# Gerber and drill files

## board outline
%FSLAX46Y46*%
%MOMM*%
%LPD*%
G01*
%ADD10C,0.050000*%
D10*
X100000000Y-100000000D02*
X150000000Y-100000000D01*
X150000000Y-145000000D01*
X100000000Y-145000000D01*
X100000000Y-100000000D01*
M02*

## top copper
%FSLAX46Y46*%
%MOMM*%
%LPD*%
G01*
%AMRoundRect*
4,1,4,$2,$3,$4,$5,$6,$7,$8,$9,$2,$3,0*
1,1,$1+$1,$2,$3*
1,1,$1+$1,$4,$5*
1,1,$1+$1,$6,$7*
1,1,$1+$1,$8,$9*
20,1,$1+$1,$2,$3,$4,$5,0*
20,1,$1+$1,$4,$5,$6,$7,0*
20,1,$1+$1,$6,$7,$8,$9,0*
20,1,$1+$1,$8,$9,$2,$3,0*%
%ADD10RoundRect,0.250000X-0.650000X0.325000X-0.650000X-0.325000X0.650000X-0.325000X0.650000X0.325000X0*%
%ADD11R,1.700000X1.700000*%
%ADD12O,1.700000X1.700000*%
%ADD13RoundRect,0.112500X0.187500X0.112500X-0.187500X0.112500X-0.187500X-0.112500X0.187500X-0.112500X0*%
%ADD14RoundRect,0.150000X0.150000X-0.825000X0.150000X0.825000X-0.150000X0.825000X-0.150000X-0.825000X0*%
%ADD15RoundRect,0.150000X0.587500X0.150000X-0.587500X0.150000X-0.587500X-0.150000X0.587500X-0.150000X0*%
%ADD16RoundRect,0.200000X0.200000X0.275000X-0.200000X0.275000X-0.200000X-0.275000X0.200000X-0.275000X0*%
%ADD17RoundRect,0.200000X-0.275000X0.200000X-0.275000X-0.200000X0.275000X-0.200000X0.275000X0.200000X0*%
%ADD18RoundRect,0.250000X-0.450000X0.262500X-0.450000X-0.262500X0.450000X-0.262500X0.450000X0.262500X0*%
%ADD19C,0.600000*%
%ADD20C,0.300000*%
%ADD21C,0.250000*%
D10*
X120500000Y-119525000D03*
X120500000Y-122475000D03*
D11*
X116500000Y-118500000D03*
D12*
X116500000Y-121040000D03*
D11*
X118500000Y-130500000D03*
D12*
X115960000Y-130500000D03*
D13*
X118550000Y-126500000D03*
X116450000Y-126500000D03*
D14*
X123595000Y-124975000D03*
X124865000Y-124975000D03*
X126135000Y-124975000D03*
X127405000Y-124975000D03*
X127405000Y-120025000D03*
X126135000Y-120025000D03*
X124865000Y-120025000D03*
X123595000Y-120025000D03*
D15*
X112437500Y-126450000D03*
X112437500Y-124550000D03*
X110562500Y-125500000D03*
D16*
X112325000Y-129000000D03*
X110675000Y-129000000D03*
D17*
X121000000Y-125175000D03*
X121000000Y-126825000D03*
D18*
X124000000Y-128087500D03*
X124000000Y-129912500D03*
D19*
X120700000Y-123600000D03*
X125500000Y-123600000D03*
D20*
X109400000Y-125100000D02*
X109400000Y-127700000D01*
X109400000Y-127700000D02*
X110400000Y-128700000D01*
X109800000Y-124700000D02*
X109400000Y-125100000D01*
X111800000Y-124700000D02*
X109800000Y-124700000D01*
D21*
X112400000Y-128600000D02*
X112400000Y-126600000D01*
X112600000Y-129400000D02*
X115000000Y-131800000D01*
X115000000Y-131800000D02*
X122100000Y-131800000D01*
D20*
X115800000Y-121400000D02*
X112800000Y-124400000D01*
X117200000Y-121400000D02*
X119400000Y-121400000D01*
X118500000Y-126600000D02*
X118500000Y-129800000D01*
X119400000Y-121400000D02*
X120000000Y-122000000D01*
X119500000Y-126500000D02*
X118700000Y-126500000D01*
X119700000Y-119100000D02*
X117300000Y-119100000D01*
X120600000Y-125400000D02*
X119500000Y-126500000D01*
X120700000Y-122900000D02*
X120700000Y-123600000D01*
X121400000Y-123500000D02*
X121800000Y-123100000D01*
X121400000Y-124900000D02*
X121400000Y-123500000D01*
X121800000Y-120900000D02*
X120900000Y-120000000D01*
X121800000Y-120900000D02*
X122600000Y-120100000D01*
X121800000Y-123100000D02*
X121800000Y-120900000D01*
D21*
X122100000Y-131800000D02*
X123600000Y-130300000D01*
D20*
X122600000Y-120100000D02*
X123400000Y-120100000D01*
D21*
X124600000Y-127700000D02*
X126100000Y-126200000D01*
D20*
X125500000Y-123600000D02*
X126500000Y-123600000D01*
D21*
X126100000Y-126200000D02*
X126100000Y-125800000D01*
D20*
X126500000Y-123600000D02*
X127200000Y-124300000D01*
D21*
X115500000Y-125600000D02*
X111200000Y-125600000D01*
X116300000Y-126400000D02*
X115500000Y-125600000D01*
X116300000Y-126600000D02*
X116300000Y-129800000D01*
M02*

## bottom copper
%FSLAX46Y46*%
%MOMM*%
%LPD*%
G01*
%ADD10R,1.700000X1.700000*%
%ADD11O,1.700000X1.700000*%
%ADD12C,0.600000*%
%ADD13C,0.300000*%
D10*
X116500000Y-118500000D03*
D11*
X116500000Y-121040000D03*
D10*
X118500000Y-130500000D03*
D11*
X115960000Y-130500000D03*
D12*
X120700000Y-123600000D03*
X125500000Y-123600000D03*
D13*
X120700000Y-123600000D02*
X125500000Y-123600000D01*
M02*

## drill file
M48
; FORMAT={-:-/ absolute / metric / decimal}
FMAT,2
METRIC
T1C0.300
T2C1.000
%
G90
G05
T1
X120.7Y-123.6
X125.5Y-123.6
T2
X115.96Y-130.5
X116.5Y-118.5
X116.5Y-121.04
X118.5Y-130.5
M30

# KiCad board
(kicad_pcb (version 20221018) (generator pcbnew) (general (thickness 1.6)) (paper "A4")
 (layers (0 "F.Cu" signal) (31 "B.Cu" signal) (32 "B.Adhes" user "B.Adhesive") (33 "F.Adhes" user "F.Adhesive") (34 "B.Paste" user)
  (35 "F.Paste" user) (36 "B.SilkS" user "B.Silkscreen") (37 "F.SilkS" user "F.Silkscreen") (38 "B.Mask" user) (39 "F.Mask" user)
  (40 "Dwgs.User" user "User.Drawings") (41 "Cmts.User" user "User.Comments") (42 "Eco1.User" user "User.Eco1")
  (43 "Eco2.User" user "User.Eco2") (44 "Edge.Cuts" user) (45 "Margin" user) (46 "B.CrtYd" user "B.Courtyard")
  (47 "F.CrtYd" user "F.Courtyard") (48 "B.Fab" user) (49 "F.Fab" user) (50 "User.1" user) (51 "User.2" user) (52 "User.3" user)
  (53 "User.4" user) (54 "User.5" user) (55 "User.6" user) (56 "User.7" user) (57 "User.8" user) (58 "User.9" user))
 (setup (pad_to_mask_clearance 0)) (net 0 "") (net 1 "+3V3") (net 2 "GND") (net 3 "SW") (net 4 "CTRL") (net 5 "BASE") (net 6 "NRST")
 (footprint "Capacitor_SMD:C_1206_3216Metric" (layer "F.Cu") (at 120.5 121 -90)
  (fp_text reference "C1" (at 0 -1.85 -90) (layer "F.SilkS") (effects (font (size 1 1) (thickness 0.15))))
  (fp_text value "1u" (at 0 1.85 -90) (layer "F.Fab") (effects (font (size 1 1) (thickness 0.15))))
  (pad "1" smd roundrect (at -1.475 0 270) (size 1.15 1.8) (layers "F.Cu" "F.Paste" "F.Mask") (roundrect_rratio 0.217391) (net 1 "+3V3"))
  (pad "2" smd roundrect (at 1.475 0 270) (size 1.15 1.8) (layers "F.Cu" "F.Paste" "F.Mask") (roundrect_rratio 0.217391) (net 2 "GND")))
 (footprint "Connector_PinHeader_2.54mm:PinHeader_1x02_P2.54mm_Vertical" (layer "F.Cu") (at 116.5 118.5)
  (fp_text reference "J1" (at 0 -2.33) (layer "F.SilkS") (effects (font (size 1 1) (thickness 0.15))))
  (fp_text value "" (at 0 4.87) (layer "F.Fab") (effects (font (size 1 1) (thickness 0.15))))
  (pad "1" thru_hole rect (at 0 0) (size 1.7 1.7) (drill 1) (layers "*.Cu" "*.Mask") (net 1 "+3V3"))
  (pad "2" thru_hole oval (at 0 2.54) (size 1.7 1.7) (drill 1) (layers "*.Cu" "*.Mask") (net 2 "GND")))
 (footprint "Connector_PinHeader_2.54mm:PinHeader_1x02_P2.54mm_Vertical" (layer "F.Cu") (at 118.5 130.5 -90)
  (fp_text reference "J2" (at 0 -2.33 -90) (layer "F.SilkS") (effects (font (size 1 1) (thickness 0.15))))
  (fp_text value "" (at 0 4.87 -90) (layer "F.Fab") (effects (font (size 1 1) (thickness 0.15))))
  (pad "1" thru_hole rect (at 0 0 270) (size 1.7 1.7) (drill 1) (layers "*.Cu" "*.Mask") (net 1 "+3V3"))
  (pad "2" thru_hole oval (at 0 2.54 270) (size 1.7 1.7) (drill 1) (layers "*.Cu" "*.Mask") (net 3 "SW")))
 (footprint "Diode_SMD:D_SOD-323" (layer "F.Cu") (at 117.5 126.5 180)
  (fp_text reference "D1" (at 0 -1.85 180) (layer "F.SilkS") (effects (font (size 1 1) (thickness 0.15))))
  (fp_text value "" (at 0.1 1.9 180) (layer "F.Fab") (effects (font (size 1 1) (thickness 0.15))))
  (pad "1" smd roundrect (at -1.05 0 180) (size 0.6 0.45) (layers "F.Cu" "F.Paste" "F.Mask") (roundrect_rratio 0.25) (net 1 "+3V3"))
  (pad "2" smd roundrect (at 1.05 0 180) (size 0.6 0.45) (layers "F.Cu" "F.Paste" "F.Mask") (roundrect_rratio 0.25) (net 3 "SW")))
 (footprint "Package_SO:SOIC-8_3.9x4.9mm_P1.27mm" (layer "F.Cu") (at 125.5 122.5 90)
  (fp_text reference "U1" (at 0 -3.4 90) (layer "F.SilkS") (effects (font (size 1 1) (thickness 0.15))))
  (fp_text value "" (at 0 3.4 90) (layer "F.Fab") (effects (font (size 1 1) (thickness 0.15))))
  (pad "1" smd roundrect (at -2.475 -1.905 90) (size 1.95 0.6) (layers "F.Cu" "F.Paste" "F.Mask") (roundrect_rratio 0.25))
  (pad "2" smd roundrect (at -2.475 -0.635 90) (size 1.95 0.6) (layers "F.Cu" "F.Paste" "F.Mask") (roundrect_rratio 0.25))
  (pad "3" smd roundrect (at -2.475 0.635 90) (size 1.95 0.6) (layers "F.Cu" "F.Paste" "F.Mask") (roundrect_rratio 0.25) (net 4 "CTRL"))
  (pad "4" smd roundrect (at -2.475 1.905 90) (size 1.95 0.6) (layers "F.Cu" "F.Paste" "F.Mask") (roundrect_rratio 0.25) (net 2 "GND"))
  (pad "5" smd roundrect (at 2.475 1.905 90) (size 1.95 0.6) (layers "F.Cu" "F.Paste" "F.Mask") (roundrect_rratio 0.25))
  (pad "6" smd roundrect (at 2.475 0.635 90) (size 1.95 0.6) (layers "F.Cu" "F.Paste" "F.Mask") (roundrect_rratio 0.25))
  (pad "7" smd roundrect (at 2.475 -0.635 90) (size 1.95 0.6) (layers "F.Cu" "F.Paste" "F.Mask") (roundrect_rratio 0.25))
  (pad "8" smd roundrect (at 2.475 -1.905 90) (size 1.95 0.6) (layers "F.Cu" "F.Paste" "F.Mask") (roundrect_rratio 0.25) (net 1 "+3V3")))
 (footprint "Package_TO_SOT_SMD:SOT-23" (layer "F.Cu") (at 111.5 125.5 180)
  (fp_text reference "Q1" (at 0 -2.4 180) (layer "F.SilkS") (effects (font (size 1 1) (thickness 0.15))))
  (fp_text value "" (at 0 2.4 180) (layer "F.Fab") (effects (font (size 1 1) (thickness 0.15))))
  (pad "1" smd roundrect (at -0.9375 -0.95 180) (size 1.475 0.6) (layers "F.Cu" "F.Paste" "F.Mask") (roundrect_rratio 0.25) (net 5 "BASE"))
  (pad "2" smd roundrect (at -0.9375 0.95 180) (size 1.475 0.6) (layers "F.Cu" "F.Paste" "F.Mask") (roundrect_rratio 0.25) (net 2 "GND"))
  (pad "3" smd roundrect (at 0.9375 0 180) (size 1.475 0.6) (layers "F.Cu" "F.Paste" "F.Mask") (roundrect_rratio 0.25) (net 3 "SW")))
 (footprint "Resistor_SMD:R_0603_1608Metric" (layer "F.Cu") (at 111.5 129 180)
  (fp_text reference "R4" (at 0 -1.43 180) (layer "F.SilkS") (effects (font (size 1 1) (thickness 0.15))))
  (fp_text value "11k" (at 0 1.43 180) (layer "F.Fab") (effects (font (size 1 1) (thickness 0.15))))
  (pad "1" smd roundrect (at -0.825 0 180) (size 0.8 0.95) (layers "F.Cu" "F.Paste" "F.Mask") (roundrect_rratio 0.25) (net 5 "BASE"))
  (pad "2" smd roundrect (at 0.825 0 180) (size 0.8 0.95) (layers "F.Cu" "F.Paste" "F.Mask") (roundrect_rratio 0.25) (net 2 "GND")))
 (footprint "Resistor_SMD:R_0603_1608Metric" (layer "F.Cu") (at 121 126 -90)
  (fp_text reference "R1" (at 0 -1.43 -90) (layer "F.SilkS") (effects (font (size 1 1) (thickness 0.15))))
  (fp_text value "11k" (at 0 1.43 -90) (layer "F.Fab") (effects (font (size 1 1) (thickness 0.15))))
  (pad "1" smd roundrect (at -0.825 0 270) (size 0.8 0.95) (layers "F.Cu" "F.Paste" "F.Mask") (roundrect_rratio 0.25) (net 1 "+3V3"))
  (pad "2" smd roundrect (at 0.825 0 270) (size 0.8 0.95) (layers "F.Cu" "F.Paste" "F.Mask") (roundrect_rratio 0.25) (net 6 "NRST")))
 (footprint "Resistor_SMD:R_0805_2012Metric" (layer "F.Cu") (at 124 129 -90)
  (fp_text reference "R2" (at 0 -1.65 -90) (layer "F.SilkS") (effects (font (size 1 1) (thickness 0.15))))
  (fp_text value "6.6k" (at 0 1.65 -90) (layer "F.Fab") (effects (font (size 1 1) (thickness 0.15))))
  (pad "1" smd roundrect (at -0.9125 0 270) (size 1.025 1.4) (layers "F.Cu" "F.Paste" "F.Mask") (roundrect_rratio 0.243902) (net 4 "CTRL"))
  (pad "2" smd roundrect (at 0.9125 0 270) (size 1.025 1.4) (layers "F.Cu" "F.Paste" "F.Mask") (roundrect_rratio 0.243902) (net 5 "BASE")))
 (gr_rect (start 100 100) (end 150 145) (stroke (width 0.05) (type default)) (fill none) (layer "Edge.Cuts"))
 (segment (start 109.4 125.1) (end 109.4 127.7) (width 0.3) (layer "F.Cu") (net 2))
 (segment (start 109.4 127.7) (end 110.4 128.7) (width 0.3) (layer "F.Cu") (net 2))
 (segment (start 109.8 124.7) (end 109.4 125.1) (width 0.3) (layer "F.Cu") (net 2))
 (segment (start 111.8 124.7) (end 109.8 124.7) (width 0.3) (layer "F.Cu") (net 2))
 (segment (start 112.4 128.6) (end 112.4 126.6) (width 0.25) (layer "F.Cu") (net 5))
 (segment (start 112.6 129.4) (end 115 131.8) (width 0.25) (layer "F.Cu") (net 5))
 (segment (start 115 131.8) (end 122.1 131.8) (width 0.25) (layer "F.Cu") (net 5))
 (segment (start 115.8 121.4) (end 112.8 124.4) (width 0.3) (layer "F.Cu") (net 2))
 (segment (start 117.2 121.4) (end 119.4 121.4) (width 0.3) (layer "F.Cu") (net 2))
 (segment (start 118.5 126.6) (end 118.5 129.8) (width 0.3) (layer "F.Cu") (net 1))
 (segment (start 119.4 121.4) (end 120 122) (width 0.3) (layer "F.Cu") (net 2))
 (segment (start 119.5 126.5) (end 118.7 126.5) (width 0.3) (layer "F.Cu") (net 1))
 (segment (start 119.7 119.1) (end 117.3 119.1) (width 0.3) (layer "F.Cu") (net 1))
 (segment (start 120.6 125.4) (end 119.5 126.5) (width 0.3) (layer "F.Cu") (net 1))
 (segment (start 120.7 122.9) (end 120.7 123.6) (width 0.3) (layer "F.Cu") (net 2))
 (segment (start 121.4 123.5) (end 121.8 123.1) (width 0.3) (layer "F.Cu") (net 1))
 (segment (start 121.4 124.9) (end 121.4 123.5) (width 0.3) (layer "F.Cu") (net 1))
 (segment (start 121.8 120.9) (end 120.9 120) (width 0.3) (layer "F.Cu") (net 1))
 (segment (start 121.8 120.9) (end 122.6 120.1) (width 0.3) (layer "F.Cu") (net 1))
 (segment (start 121.8 123.1) (end 121.8 120.9) (width 0.3) (layer "F.Cu") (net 1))
 (segment (start 122.1 131.8) (end 123.6 130.3) (width 0.25) (layer "F.Cu") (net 5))
 (segment (start 122.6 120.1) (end 123.4 120.1) (width 0.3) (layer "F.Cu") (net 1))
 (segment (start 124.6 127.7) (end 126.1 126.2) (width 0.25) (layer "F.Cu") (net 4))
 (segment (start 125.5 123.6) (end 126.5 123.6) (width 0.3) (layer "F.Cu") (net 2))
 (segment (start 126.1 126.2) (end 126.1 125.8) (width 0.25) (layer "F.Cu") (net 4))
 (segment (start 126.5 123.6) (end 127.2 124.3) (width 0.3) (layer "F.Cu") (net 2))
 (via (at 120.7 123.6) (size 0.6) (drill 0.3) (layers "F.Cu" "B.Cu") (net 2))
 (via (at 125.5 123.6) (size 0.6) (drill 0.3) (layers "F.Cu" "B.Cu") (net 2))
 (segment (start 115.5 125.6) (end 111.2 125.6) (width 0.25) (layer "F.Cu") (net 3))
 (segment (start 116.3 126.4) (end 115.5 125.6) (width 0.25) (layer "F.Cu") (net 3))
 (segment (start 116.3 126.6) (end 116.3 129.8) (width 0.25) (layer "F.Cu") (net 3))
 (segment (start 120.7 123.6) (end 125.5 123.6) (width 0.3) (layer "B.Cu") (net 2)))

